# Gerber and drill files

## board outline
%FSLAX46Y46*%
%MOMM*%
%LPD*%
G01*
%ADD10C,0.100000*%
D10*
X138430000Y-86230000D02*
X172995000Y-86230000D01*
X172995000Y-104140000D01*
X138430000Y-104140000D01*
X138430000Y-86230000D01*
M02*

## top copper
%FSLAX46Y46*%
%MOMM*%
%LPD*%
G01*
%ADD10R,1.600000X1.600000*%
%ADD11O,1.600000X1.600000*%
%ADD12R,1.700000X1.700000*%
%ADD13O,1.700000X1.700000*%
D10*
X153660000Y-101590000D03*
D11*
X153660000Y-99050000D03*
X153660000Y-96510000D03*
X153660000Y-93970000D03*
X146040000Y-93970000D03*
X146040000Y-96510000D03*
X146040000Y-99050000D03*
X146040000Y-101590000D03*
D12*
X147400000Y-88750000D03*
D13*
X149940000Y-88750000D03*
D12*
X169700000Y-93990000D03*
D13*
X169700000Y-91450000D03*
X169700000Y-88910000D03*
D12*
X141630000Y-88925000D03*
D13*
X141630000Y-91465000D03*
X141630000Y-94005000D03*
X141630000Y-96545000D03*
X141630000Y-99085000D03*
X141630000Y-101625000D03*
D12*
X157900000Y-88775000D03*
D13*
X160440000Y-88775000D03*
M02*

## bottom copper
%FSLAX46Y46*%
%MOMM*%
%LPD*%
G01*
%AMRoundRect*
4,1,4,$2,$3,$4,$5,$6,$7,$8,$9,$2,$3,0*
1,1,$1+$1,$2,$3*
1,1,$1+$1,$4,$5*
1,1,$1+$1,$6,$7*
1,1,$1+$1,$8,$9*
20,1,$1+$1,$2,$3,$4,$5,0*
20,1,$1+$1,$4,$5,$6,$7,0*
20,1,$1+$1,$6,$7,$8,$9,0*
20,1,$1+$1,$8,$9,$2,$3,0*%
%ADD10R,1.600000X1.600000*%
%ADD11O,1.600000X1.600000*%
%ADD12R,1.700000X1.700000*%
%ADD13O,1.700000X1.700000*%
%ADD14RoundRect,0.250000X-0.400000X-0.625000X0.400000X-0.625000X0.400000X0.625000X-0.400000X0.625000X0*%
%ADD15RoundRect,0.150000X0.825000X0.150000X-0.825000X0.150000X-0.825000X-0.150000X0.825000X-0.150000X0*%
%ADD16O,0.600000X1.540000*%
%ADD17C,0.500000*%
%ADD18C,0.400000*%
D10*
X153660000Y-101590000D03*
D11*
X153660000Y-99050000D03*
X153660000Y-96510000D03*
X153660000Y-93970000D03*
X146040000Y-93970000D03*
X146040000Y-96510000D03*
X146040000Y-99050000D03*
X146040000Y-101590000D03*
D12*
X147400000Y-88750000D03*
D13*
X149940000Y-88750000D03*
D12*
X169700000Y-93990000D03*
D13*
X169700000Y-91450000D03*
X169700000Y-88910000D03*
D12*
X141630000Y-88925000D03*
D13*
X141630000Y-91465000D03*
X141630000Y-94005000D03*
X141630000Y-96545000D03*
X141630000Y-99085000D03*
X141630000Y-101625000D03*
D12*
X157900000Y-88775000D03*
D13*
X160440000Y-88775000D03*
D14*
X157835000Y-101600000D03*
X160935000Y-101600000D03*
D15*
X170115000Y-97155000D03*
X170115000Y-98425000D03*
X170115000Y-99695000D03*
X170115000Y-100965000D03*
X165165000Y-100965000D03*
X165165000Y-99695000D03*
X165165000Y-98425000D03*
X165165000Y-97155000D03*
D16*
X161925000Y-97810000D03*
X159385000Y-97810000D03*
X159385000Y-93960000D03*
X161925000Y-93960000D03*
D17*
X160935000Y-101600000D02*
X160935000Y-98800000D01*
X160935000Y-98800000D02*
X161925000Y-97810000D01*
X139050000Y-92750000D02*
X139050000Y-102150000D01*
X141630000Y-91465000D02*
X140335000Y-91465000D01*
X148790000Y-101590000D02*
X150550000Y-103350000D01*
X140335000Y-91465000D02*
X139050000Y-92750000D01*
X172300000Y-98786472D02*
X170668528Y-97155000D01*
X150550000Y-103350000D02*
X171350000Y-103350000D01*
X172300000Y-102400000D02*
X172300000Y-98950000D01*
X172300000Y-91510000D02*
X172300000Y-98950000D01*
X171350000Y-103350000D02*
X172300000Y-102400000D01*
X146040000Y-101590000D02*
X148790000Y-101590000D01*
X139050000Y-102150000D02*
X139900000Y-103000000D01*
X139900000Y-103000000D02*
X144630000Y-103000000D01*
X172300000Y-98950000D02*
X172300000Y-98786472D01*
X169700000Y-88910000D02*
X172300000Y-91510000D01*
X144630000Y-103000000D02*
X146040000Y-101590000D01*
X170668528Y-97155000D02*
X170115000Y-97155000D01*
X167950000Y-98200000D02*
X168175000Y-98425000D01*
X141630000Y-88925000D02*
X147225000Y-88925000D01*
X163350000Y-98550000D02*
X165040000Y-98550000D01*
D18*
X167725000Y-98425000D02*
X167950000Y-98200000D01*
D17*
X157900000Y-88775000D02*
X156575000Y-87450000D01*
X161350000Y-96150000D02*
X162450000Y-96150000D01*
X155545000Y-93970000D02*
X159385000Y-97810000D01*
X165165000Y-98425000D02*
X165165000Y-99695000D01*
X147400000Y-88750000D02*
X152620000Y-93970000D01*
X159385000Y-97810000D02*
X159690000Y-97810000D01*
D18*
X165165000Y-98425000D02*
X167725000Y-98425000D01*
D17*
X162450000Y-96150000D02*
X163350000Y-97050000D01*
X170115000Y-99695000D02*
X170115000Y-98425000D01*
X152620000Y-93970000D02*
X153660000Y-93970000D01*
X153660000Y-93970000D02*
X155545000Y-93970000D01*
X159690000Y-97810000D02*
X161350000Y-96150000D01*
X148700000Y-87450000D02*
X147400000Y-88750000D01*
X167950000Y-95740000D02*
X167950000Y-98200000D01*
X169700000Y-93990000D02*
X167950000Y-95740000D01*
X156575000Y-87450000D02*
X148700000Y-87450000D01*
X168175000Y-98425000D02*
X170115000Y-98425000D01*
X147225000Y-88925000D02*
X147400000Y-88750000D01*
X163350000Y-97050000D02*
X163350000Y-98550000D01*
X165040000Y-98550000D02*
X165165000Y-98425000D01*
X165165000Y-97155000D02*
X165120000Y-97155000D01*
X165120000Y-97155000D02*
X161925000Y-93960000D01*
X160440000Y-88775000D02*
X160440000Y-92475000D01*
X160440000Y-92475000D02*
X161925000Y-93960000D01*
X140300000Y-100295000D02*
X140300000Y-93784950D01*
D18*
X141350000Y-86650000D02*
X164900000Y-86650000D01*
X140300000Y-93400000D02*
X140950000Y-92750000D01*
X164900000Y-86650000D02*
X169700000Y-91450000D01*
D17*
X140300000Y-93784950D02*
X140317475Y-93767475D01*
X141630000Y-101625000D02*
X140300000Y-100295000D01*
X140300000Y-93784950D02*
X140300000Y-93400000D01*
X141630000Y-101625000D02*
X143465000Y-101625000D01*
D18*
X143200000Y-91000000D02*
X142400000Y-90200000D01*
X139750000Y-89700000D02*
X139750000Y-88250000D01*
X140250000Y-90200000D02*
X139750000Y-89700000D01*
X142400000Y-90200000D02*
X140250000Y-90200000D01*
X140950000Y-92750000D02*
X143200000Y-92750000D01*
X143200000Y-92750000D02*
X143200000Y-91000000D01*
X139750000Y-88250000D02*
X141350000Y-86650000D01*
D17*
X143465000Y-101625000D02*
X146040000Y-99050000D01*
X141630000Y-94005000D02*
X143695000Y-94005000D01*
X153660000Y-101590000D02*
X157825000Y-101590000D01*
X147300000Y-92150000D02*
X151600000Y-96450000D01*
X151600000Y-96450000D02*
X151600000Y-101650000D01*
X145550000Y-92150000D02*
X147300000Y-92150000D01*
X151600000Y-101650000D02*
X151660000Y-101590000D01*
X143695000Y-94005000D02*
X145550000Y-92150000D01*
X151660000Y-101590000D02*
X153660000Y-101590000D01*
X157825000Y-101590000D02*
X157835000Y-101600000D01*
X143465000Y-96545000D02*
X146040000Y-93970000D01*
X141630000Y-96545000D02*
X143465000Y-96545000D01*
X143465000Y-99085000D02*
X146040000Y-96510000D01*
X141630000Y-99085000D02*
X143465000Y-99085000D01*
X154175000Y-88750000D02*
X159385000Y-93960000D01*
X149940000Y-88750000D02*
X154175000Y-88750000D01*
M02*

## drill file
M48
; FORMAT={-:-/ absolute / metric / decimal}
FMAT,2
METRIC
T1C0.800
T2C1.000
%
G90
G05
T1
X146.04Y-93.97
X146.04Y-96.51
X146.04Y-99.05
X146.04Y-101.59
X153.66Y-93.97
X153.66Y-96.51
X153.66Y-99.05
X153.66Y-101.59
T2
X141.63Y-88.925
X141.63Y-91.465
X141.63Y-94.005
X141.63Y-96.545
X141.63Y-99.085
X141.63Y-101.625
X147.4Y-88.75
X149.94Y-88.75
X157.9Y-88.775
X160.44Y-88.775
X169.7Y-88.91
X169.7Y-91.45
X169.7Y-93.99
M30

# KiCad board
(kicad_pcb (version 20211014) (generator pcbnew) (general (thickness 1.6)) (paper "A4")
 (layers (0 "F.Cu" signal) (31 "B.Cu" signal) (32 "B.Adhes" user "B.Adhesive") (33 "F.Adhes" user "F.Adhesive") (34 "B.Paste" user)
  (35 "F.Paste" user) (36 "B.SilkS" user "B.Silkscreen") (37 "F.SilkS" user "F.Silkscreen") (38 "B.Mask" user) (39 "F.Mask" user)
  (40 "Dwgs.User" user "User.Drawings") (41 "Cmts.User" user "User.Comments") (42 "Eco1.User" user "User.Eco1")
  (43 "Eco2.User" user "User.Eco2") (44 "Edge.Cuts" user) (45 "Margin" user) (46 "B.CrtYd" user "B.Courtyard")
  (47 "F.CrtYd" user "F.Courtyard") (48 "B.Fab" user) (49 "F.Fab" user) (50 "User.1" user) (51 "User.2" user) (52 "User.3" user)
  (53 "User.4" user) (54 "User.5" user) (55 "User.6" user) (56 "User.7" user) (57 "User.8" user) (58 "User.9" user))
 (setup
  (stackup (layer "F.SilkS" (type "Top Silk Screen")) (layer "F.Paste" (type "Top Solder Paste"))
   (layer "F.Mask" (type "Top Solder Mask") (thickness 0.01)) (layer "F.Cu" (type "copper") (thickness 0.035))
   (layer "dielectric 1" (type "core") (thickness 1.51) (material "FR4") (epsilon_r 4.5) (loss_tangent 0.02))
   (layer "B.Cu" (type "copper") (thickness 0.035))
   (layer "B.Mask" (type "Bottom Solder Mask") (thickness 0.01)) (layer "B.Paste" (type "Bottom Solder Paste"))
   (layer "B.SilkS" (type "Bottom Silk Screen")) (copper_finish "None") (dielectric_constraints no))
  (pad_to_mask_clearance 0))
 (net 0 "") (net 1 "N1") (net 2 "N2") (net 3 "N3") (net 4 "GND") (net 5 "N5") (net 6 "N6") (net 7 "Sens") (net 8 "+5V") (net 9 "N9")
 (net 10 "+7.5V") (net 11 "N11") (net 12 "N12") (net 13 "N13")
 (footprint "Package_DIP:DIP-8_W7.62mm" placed (layer "F.Cu") (at 153.66 101.59 180)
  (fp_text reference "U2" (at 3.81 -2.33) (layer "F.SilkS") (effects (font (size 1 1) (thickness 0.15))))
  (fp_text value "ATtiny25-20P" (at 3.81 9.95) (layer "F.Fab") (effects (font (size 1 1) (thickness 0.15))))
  (pad "1" thru_hole rect locked (at 0 0 180) (size 1.6 1.6) (drill 0.8) (layers *.Cu *.Mask) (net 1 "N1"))
  (pad "2" thru_hole oval locked (at 0 2.54 180) (size 1.6 1.6) (drill 0.8) (layers *.Cu *.Mask) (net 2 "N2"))
  (pad "3" thru_hole oval locked (at 0 5.08 180) (size 1.6 1.6) (drill 0.8) (layers *.Cu *.Mask) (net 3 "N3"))
  (pad "4" thru_hole oval locked (at 0 7.62 180) (size 1.6 1.6) (drill 0.8) (layers *.Cu *.Mask) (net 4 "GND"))
  (pad "5" thru_hole oval locked (at 7.62 7.62 180) (size 1.6 1.6) (drill 0.8) (layers *.Cu *.Mask) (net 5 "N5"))
  (pad "6" thru_hole oval locked (at 7.62 5.08 180) (size 1.6 1.6) (drill 0.8) (layers *.Cu *.Mask) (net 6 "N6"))
  (pad "7" thru_hole oval locked (at 7.62 2.54 180) (size 1.6 1.6) (drill 0.8) (layers *.Cu *.Mask) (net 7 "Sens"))
  (pad "8" thru_hole oval locked (at 7.62 0 180) (size 1.6 1.6) (drill 0.8) (layers *.Cu *.Mask) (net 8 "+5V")))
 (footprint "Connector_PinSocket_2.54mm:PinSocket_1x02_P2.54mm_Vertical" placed (layer "F.Cu") (at 147.4 88.75 90)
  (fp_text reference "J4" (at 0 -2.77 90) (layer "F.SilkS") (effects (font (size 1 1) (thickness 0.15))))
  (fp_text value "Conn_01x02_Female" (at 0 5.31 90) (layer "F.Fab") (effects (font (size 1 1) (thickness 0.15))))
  (pad "1" thru_hole rect locked (at 0 0 90) (size 1.7 1.7) (drill 1) (layers *.Cu *.Mask) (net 4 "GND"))
  (pad "2" thru_hole oval locked (at 0 2.54 90) (size 1.7 1.7) (drill 1) (layers *.Cu *.Mask) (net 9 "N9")))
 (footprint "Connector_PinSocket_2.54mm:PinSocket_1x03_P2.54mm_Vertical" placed (layer "F.Cu") (at 169.7 93.99 180)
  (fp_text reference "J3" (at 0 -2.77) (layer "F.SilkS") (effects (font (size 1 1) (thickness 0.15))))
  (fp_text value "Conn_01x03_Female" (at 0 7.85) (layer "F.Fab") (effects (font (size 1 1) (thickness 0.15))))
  (pad "1" thru_hole rect locked (at 0 0 180) (size 1.7 1.7) (drill 1) (layers *.Cu *.Mask) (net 4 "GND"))
  (pad "2" thru_hole oval locked (at 0 2.54 180) (size 1.7 1.7) (drill 1) (layers *.Cu *.Mask) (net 7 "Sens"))
  (pad "3" thru_hole oval locked (at 0 5.08 180) (size 1.7 1.7) (drill 1) (layers *.Cu *.Mask) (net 8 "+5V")))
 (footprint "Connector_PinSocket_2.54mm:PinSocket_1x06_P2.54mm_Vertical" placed (layer "F.Cu") (at 141.63 88.925)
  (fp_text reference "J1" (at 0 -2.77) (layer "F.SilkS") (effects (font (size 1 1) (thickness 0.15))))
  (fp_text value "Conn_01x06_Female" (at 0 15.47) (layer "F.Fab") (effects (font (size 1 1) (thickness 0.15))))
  (pad "1" thru_hole rect locked (at 0 0) (size 1.7 1.7) (drill 1) (layers *.Cu *.Mask) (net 4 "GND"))
  (pad "2" thru_hole oval locked (at 0 2.54) (size 1.7 1.7) (drill 1) (layers *.Cu *.Mask) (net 8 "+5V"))
  (pad "3" thru_hole oval locked (at 0 5.08) (size 1.7 1.7) (drill 1) (layers *.Cu *.Mask) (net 1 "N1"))
  (pad "4" thru_hole oval locked (at 0 7.62) (size 1.7 1.7) (drill 1) (layers *.Cu *.Mask) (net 5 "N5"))
  (pad "5" thru_hole oval locked (at 0 10.16) (size 1.7 1.7) (drill 1) (layers *.Cu *.Mask) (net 6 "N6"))
  (pad "6" thru_hole oval locked (at 0 12.7) (size 1.7 1.7) (drill 1) (layers *.Cu *.Mask) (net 7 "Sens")))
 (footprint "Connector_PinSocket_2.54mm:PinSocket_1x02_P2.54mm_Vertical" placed (layer "F.Cu") (at 157.9 88.775 90)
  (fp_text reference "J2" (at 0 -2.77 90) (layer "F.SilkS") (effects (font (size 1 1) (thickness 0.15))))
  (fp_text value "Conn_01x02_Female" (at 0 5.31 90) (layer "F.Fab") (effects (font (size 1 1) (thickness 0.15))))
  (pad "1" thru_hole rect locked (at 0 0 90) (size 1.7 1.7) (drill 1) (layers *.Cu *.Mask) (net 4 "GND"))
  (pad "2" thru_hole oval locked (at 0 2.54 90) (size 1.7 1.7) (drill 1) (layers *.Cu *.Mask) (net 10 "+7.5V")))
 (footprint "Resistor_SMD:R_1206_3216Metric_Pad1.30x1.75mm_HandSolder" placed (layer "B.Cu") (at 159.385 101.6)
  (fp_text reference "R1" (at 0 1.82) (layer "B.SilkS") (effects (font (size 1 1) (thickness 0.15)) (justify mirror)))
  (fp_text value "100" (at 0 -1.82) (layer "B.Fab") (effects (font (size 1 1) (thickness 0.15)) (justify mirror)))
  (pad "1" smd roundrect locked (at -1.55 0) (size 1.3 1.75) (layers "B.Cu" "B.Paste" "B.Mask") (roundrect_rratio 0.1923076923) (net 1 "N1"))
  (pad "2" smd roundrect locked (at 1.55 0) (size 1.3 1.75) (layers "B.Cu" "B.Paste" "B.Mask") (roundrect_rratio 0.1923076923)
   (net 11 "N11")))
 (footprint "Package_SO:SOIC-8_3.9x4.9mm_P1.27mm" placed (layer "B.Cu") (at 167.64 99.06 180)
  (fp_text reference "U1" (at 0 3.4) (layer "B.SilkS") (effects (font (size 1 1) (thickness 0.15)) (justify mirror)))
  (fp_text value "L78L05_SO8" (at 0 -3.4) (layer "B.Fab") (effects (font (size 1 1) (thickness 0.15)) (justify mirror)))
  (pad "1" smd roundrect locked (at -2.475 1.905 180) (size 1.95 0.6) (layers "B.Cu" "B.Paste" "B.Mask") (roundrect_rratio 0.25)
   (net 8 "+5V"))
  (pad "2" smd roundrect locked (at -2.475 0.635 180) (size 1.95 0.6) (layers "B.Cu" "B.Paste" "B.Mask") (roundrect_rratio 0.25)
   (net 4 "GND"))
  (pad "3" smd roundrect locked (at -2.475 -0.635 180) (size 1.95 0.6) (layers "B.Cu" "B.Paste" "B.Mask") (roundrect_rratio 0.25)
   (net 4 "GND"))
  (pad "4" smd roundrect locked (at -2.475 -1.905 180) (size 1.95 0.6) (layers "B.Cu" "B.Paste" "B.Mask") (roundrect_rratio 0.25)
   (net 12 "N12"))
  (pad "5" smd roundrect locked (at 2.475 -1.905 180) (size 1.95 0.6) (layers "B.Cu" "B.Paste" "B.Mask") (roundrect_rratio 0.25)
   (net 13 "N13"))
  (pad "6" smd roundrect locked (at 2.475 -0.635 180) (size 1.95 0.6) (layers "B.Cu" "B.Paste" "B.Mask") (roundrect_rratio 0.25)
   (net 4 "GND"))
  (pad "7" smd roundrect locked (at 2.475 0.635 180) (size 1.95 0.6) (layers "B.Cu" "B.Paste" "B.Mask") (roundrect_rratio 0.25)
   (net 4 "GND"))
  (pad "8" smd roundrect locked (at 2.475 1.905 180) (size 1.95 0.6) (layers "B.Cu" "B.Paste" "B.Mask") (roundrect_rratio 0.25)
   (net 10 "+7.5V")))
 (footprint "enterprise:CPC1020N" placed (layer "B.Cu") (at 161.925 93.96 180)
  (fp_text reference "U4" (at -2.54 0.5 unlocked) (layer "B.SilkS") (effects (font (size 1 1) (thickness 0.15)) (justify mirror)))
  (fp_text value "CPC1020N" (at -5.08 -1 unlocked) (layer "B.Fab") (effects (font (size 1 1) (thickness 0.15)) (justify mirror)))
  (pad "1" smd oval (at 0 -3.85 90) (size 1.54 0.6) (layers "B.Cu" "B.Paste" "B.Mask") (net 11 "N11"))
  (pad "2" smd oval (at 2.54 -3.85 90) (size 1.54 0.6) (layers "B.Cu" "B.Paste" "B.Mask") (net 4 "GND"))
  (pad "3" smd oval (at 2.54 0 90) (size 1.54 0.6) (layers "B.Cu" "B.Paste" "B.Mask") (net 9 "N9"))
  (pad "4" smd oval (at 0 0 90) (size 1.54 0.6) (layers "B.Cu" "B.Paste" "B.Mask") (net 10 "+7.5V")))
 (gr_rect (start 138.43 86.23) (end 172.995 104.14) (layer "Edge.Cuts") (width 0.1) (fill none))
 (segment (start 160.935 101.6) (end 160.935 98.8) (width 0.5) (layer "B.Cu") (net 11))
 (segment (start 160.935 98.8) (end 161.925 97.81) (width 0.5) (layer "B.Cu") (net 11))
 (segment (start 139.05 92.75) (end 139.05 102.15) (width 0.5) (layer "B.Cu") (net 8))
 (segment (start 141.63 91.465) (end 140.335 91.465) (width 0.5) (layer "B.Cu") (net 8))
 (segment (start 148.79 101.59) (end 150.55 103.35) (width 0.5) (layer "B.Cu") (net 8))
 (segment (start 140.335 91.465) (end 139.05 92.75) (width 0.5) (layer "B.Cu") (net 8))
 (segment (start 172.3 98.786472) (end 170.668528 97.155) (width 0.5) (layer "B.Cu") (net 8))
 (segment (start 150.55 103.35) (end 171.35 103.35) (width 0.5) (layer "B.Cu") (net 8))
 (segment (start 172.3 102.4) (end 172.3 98.95) (width 0.5) (layer "B.Cu") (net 8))
 (segment (start 172.3 91.51) (end 172.3 98.95) (width 0.5) (layer "B.Cu") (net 8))
 (segment (start 171.35 103.35) (end 172.3 102.4) (width 0.5) (layer "B.Cu") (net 8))
 (segment (start 146.04 101.59) (end 148.79 101.59) (width 0.5) (layer "B.Cu") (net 8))
 (segment (start 139.05 102.15) (end 139.9 103) (width 0.5) (layer "B.Cu") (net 8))
 (segment (start 139.9 103) (end 144.63 103) (width 0.5) (layer "B.Cu") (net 8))
 (segment (start 172.3 98.95) (end 172.3 98.786472) (width 0.5) (layer "B.Cu") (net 8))
 (segment (start 169.7 88.91) (end 172.3 91.51) (width 0.5) (layer "B.Cu") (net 8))
 (segment (start 144.63 103) (end 146.04 101.59) (width 0.5) (layer "B.Cu") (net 8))
 (segment (start 170.668528 97.155) (end 170.115 97.155) (width 0.5) (layer "B.Cu") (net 8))
 (segment (start 167.95 98.2) (end 168.175 98.425) (width 0.5) (layer "B.Cu") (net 4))
 (segment (start 141.63 88.925) (end 147.225 88.925) (width 0.5) (layer "B.Cu") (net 4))
 (segment (start 163.35 98.55) (end 165.04 98.55) (width 0.5) (layer "B.Cu") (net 4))
 (segment (start 167.725 98.425) (end 167.95 98.2) (width 0.4) (layer "B.Cu") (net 4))
 (segment (start 157.9 88.775) (end 156.575 87.45) (width 0.5) (layer "B.Cu") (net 4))
 (segment (start 161.35 96.15) (end 162.45 96.15) (width 0.5) (layer "B.Cu") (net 4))
 (segment (start 155.545 93.97) (end 159.385 97.81) (width 0.5) (layer "B.Cu") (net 4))
 (segment (start 165.165 98.425) (end 165.165 99.695) (width 0.5) (layer "B.Cu") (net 4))
 (segment (start 147.4 88.75) (end 152.62 93.97) (width 0.5) (layer "B.Cu") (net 4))
 (segment (start 159.385 97.81) (end 159.69 97.81) (width 0.5) (layer "B.Cu") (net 4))
 (segment (start 165.165 98.425) (end 167.725 98.425) (width 0.4) (layer "B.Cu") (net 4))
 (segment (start 162.45 96.15) (end 163.35 97.05) (width 0.5) (layer "B.Cu") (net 4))
 (segment (start 170.115 99.695) (end 170.115 98.425) (width 0.5) (layer "B.Cu") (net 4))
 (segment (start 152.62 93.97) (end 153.66 93.97) (width 0.5) (layer "B.Cu") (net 4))
 (segment (start 153.66 93.97) (end 155.545 93.97) (width 0.5) (layer "B.Cu") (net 4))
 (segment (start 159.69 97.81) (end 161.35 96.15) (width 0.5) (layer "B.Cu") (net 4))
 (segment (start 148.7 87.45) (end 147.4 88.75) (width 0.5) (layer "B.Cu") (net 4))
 (segment (start 167.95 95.74) (end 167.95 98.2) (width 0.5) (layer "B.Cu") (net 4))
 (segment (start 169.7 93.99) (end 167.95 95.74) (width 0.5) (layer "B.Cu") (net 4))
 (segment (start 156.575 87.45) (end 148.7 87.45) (width 0.5) (layer "B.Cu") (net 4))
 (segment (start 168.175 98.425) (end 170.115 98.425) (width 0.5) (layer "B.Cu") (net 4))
 (segment (start 147.225 88.925) (end 147.4 88.75) (width 0.5) (layer "B.Cu") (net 4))
 (segment (start 163.35 97.05) (end 163.35 98.55) (width 0.5) (layer "B.Cu") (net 4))
 (segment (start 165.04 98.55) (end 165.165 98.425) (width 0.5) (layer "B.Cu") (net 4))
 (segment (start 165.165 97.155) (end 165.12 97.155) (width 0.5) (layer "B.Cu") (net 10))
 (segment (start 165.12 97.155) (end 161.925 93.96) (width 0.5) (layer "B.Cu") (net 10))
 (segment (start 160.44 88.775) (end 160.44 92.475) (width 0.5) (layer "B.Cu") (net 10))
 (segment (start 160.44 92.475) (end 161.925 93.96) (width 0.5) (layer "B.Cu") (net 10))
 (segment (start 140.3 100.295) (end 140.3 93.78495) (width 0.5) (layer "B.Cu") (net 7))
 (segment (start 141.35 86.65) (end 164.9 86.65) (width 0.4) (layer "B.Cu") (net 7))
 (segment (start 140.3 93.4) (end 140.95 92.75) (width 0.4) (layer "B.Cu") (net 7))
 (segment (start 164.9 86.65) (end 169.7 91.45) (width 0.4) (layer "B.Cu") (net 7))
 (segment (start 140.3 93.78495) (end 140.317475 93.767475) (width 0.5) (layer "B.Cu") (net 7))
 (segment (start 141.63 101.625) (end 140.3 100.295) (width 0.5) (layer "B.Cu") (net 7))
 (segment (start 140.3 93.78495) (end 140.3 93.4) (width 0.5) (layer "B.Cu") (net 7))
 (segment (start 141.63 101.625) (end 143.465 101.625) (width 0.5) (layer "B.Cu") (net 7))
 (segment (start 143.2 91) (end 142.4 90.2) (width 0.4) (layer "B.Cu") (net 7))
 (segment (start 139.75 89.7) (end 139.75 88.25) (width 0.4) (layer "B.Cu") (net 7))
 (segment (start 140.25 90.2) (end 139.75 89.7) (width 0.4) (layer "B.Cu") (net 7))
 (segment (start 142.4 90.2) (end 140.25 90.2) (width 0.4) (layer "B.Cu") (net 7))
 (segment (start 140.95 92.75) (end 143.2 92.75) (width 0.4) (layer "B.Cu") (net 7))
 (segment (start 143.2 92.75) (end 143.2 91) (width 0.4) (layer "B.Cu") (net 7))
 (segment (start 139.75 88.25) (end 141.35 86.65) (width 0.4) (layer "B.Cu") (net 7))
 (segment (start 143.465 101.625) (end 146.04 99.05) (width 0.5) (layer "B.Cu") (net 7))
 (segment (start 141.63 94.005) (end 143.695 94.005) (width 0.5) (layer "B.Cu") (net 1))
 (segment (start 153.66 101.59) (end 157.825 101.59) (width 0.5) (layer "B.Cu") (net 1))
 (segment (start 147.3 92.15) (end 151.6 96.45) (width 0.5) (layer "B.Cu") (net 1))
 (segment (start 151.6 96.45) (end 151.6 101.65) (width 0.5) (layer "B.Cu") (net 1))
 (segment (start 145.55 92.15) (end 147.3 92.15) (width 0.5) (layer "B.Cu") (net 1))
 (segment (start 151.6 101.65) (end 151.66 101.59) (width 0.5) (layer "B.Cu") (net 1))
 (segment (start 143.695 94.005) (end 145.55 92.15) (width 0.5) (layer "B.Cu") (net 1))
 (segment (start 151.66 101.59) (end 153.66 101.59) (width 0.5) (layer "B.Cu") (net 1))
 (segment (start 157.825 101.59) (end 157.835 101.6) (width 0.5) (layer "B.Cu") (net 1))
 (segment (start 143.465 96.545) (end 146.04 93.97) (width 0.5) (layer "B.Cu") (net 5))
 (segment (start 141.63 96.545) (end 143.465 96.545) (width 0.5) (layer "B.Cu") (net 5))
 (segment (start 143.465 99.085) (end 146.04 96.51) (width 0.5) (layer "B.Cu") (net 6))
 (segment (start 141.63 99.085) (end 143.465 99.085) (width 0.5) (layer "B.Cu") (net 6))
 (segment (start 154.175 88.75) (end 159.385 93.96) (width 0.5) (layer "B.Cu") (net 9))
 (segment (start 149.94 88.75) (end 154.175 88.75) (width 0.5) (layer "B.Cu") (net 9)))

